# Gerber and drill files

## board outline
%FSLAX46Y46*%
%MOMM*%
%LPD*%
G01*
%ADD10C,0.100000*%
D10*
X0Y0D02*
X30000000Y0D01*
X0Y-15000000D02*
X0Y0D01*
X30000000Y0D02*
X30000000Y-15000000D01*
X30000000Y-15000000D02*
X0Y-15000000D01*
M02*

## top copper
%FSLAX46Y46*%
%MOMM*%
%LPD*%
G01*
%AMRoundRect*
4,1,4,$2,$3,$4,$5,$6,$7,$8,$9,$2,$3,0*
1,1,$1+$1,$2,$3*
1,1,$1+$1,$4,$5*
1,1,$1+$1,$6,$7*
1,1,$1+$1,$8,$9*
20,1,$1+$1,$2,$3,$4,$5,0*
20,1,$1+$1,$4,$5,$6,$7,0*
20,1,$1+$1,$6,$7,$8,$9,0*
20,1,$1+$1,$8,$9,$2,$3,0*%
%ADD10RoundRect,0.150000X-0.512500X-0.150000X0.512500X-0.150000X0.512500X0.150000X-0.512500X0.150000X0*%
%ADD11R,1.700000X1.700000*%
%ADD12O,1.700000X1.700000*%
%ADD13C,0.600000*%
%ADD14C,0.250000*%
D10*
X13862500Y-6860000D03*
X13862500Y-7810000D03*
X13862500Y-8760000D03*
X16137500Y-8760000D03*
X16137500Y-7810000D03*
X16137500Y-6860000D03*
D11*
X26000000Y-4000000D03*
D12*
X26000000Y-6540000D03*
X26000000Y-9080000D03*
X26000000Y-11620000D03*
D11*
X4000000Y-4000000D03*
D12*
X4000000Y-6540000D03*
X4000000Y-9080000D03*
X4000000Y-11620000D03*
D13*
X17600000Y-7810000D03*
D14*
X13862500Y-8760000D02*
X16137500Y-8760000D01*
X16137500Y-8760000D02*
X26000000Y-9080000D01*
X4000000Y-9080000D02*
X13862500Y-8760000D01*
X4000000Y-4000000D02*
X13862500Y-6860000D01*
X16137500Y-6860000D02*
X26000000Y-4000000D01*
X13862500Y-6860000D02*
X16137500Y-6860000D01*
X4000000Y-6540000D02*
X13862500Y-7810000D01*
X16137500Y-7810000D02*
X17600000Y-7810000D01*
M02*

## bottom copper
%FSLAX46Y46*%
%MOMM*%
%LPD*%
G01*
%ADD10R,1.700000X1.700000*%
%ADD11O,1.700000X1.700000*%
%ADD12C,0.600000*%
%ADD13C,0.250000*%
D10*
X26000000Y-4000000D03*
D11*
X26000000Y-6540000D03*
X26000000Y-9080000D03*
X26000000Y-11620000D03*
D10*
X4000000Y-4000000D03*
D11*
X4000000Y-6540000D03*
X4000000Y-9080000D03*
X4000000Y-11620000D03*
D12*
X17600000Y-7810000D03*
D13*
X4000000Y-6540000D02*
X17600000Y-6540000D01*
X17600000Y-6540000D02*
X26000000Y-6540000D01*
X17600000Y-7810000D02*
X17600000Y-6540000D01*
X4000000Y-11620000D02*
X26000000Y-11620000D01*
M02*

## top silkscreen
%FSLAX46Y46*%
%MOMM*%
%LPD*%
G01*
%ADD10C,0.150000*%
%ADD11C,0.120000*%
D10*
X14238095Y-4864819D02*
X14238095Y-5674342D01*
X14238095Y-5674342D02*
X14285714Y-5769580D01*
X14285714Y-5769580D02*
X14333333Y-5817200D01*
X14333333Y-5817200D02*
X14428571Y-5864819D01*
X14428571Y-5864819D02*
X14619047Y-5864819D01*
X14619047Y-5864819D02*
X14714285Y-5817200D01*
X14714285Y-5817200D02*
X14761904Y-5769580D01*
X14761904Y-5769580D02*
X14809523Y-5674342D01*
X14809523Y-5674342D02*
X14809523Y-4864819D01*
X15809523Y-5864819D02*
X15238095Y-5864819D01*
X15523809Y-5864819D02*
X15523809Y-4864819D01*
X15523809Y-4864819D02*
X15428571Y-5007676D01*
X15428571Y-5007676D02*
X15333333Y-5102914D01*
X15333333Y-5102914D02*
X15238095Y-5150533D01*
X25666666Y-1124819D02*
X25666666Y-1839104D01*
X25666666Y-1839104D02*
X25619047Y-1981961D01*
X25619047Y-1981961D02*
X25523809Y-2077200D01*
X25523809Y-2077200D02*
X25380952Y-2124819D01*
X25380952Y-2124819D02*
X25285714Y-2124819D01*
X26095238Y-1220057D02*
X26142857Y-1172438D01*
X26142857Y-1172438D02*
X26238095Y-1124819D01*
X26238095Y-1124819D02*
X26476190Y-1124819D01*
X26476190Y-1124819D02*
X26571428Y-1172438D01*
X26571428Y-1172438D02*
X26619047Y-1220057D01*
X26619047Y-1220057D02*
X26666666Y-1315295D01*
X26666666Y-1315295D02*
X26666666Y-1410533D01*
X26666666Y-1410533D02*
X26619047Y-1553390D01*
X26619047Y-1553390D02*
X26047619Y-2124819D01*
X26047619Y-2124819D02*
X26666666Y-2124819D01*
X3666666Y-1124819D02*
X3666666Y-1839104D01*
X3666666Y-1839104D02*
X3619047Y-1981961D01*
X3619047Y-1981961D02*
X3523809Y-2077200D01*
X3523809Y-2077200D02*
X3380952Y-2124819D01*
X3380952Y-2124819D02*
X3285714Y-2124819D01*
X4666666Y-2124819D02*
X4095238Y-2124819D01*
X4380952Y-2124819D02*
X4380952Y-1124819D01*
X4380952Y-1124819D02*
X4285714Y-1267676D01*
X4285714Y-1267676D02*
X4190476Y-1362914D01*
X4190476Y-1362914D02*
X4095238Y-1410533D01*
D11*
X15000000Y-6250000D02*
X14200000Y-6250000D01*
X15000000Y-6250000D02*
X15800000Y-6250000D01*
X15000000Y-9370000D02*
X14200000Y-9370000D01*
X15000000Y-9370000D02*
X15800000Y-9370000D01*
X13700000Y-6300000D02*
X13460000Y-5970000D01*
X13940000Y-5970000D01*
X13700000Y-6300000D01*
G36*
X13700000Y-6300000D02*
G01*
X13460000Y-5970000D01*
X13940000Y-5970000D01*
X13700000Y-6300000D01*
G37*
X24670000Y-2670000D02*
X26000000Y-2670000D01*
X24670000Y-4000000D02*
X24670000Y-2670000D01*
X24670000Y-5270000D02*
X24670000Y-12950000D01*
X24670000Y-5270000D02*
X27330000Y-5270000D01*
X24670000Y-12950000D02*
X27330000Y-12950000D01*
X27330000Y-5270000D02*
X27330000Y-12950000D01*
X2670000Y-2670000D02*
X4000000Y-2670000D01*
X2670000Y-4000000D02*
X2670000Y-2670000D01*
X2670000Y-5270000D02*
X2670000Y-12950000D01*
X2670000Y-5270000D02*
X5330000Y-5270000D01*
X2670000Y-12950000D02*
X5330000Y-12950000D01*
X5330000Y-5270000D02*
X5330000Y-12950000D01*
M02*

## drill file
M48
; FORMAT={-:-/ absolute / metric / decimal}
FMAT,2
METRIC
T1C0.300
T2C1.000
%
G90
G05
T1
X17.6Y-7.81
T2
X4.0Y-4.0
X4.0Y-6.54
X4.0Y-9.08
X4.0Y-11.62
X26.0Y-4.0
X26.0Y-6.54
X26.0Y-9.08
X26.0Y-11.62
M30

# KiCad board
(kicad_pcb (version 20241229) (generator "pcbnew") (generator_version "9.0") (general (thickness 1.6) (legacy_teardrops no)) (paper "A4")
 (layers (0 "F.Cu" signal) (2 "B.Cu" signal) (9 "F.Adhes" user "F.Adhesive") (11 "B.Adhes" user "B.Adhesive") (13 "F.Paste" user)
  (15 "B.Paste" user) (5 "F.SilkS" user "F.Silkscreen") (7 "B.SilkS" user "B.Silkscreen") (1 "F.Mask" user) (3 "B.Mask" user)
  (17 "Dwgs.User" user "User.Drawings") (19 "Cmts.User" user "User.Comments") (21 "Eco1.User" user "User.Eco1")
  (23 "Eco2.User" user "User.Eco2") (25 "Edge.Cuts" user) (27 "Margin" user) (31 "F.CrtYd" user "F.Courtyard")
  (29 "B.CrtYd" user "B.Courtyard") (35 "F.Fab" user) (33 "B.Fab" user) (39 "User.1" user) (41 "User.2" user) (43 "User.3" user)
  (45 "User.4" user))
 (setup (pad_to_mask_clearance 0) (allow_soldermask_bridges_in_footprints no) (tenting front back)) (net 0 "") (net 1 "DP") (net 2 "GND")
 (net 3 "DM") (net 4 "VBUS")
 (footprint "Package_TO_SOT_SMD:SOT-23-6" (layer "F.Cu") (at 15 7.81)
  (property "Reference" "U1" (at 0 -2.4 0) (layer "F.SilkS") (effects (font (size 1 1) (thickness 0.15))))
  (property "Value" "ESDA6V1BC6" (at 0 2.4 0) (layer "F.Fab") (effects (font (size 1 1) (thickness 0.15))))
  (fp_line (start 0 -1.56) (end -0.8 -1.56) (stroke (width 0.12) (type solid)) (layer "F.SilkS"))
  (fp_line (start 0 -1.56) (end 0.8 -1.56) (stroke (width 0.12) (type solid)) (layer "F.SilkS"))
  (fp_line (start 0 1.56) (end -0.8 1.56) (stroke (width 0.12) (type solid)) (layer "F.SilkS"))
  (fp_line (start 0 1.56) (end 0.8 1.56) (stroke (width 0.12) (type solid)) (layer "F.SilkS"))
  (fp_poly
   (pts (xy -1.3 -1.51) (xy -1.54 -1.84) (xy -1.06 -1.84) (xy -1.3 -1.51)) (stroke (width 0.12) (type solid)) (fill yes) (layer "F.SilkS"))
  (pad "1" smd roundrect (at -1.1375 -0.95) (size 1.325 0.6) (layers "F.Cu" "F.Mask" "F.Paste") (roundrect_rratio 0.25) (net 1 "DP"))
  (pad "2" smd roundrect (at -1.1375 0) (size 1.325 0.6) (layers "F.Cu" "F.Mask" "F.Paste") (roundrect_rratio 0.25) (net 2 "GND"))
  (pad "3" smd roundrect (at -1.1375 0.95) (size 1.325 0.6) (layers "F.Cu" "F.Mask" "F.Paste") (roundrect_rratio 0.25) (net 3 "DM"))
  (pad "4" smd roundrect (at 1.1375 0.95) (size 1.325 0.6) (layers "F.Cu" "F.Mask" "F.Paste") (roundrect_rratio 0.25) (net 3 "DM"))
  (pad "5" smd roundrect (at 1.1375 0) (size 1.325 0.6) (layers "F.Cu" "F.Mask" "F.Paste") (roundrect_rratio 0.25) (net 2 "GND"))
  (pad "6" smd roundrect (at 1.1375 -0.95) (size 1.325 0.6) (layers "F.Cu" "F.Mask" "F.Paste") (roundrect_rratio 0.25) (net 1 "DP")))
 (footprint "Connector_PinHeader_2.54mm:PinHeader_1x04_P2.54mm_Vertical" (layer "F.Cu") (at 26 4)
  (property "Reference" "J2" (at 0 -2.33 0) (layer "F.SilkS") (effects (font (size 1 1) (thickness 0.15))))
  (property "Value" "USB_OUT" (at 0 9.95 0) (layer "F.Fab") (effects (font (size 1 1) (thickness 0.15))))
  (fp_line (start -1.33 -1.33) (end 0 -1.33) (stroke (width 0.12) (type solid)) (layer "F.SilkS"))
  (fp_line (start -1.33 0) (end -1.33 -1.33) (stroke (width 0.12) (type solid)) (layer "F.SilkS"))
  (fp_line (start -1.33 1.27) (end -1.33 8.95) (stroke (width 0.12) (type solid)) (layer "F.SilkS"))
  (fp_line (start -1.33 1.27) (end 1.33 1.27) (stroke (width 0.12) (type solid)) (layer "F.SilkS"))
  (fp_line (start -1.33 8.95) (end 1.33 8.95) (stroke (width 0.12) (type solid)) (layer "F.SilkS"))
  (fp_line (start 1.33 1.27) (end 1.33 8.95) (stroke (width 0.12) (type solid)) (layer "F.SilkS"))
  (pad "1" thru_hole rect (at 0 0) (size 1.7 1.7) (drill 1) (layers "*.Cu" "*.Mask") (remove_unused_layers no) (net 1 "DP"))
  (pad "2" thru_hole oval (at 0 2.54) (size 1.7 1.7) (drill 1) (layers "*.Cu" "*.Mask") (remove_unused_layers no) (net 2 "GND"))
  (pad "3" thru_hole oval (at 0 5.08) (size 1.7 1.7) (drill 1) (layers "*.Cu" "*.Mask") (remove_unused_layers no) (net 3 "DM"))
  (pad "4" thru_hole oval (at 0 7.62) (size 1.7 1.7) (drill 1) (layers "*.Cu" "*.Mask") (remove_unused_layers no) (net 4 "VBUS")))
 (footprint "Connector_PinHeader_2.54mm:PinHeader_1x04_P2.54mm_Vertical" (layer "F.Cu") (at 4 4)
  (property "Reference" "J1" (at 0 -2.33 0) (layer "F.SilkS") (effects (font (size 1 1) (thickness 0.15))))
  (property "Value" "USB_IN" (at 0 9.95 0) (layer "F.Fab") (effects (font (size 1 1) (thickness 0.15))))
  (fp_line (start -1.33 -1.33) (end 0 -1.33) (stroke (width 0.12) (type solid)) (layer "F.SilkS"))
  (fp_line (start -1.33 0) (end -1.33 -1.33) (stroke (width 0.12) (type solid)) (layer "F.SilkS"))
  (fp_line (start -1.33 1.27) (end -1.33 8.95) (stroke (width 0.12) (type solid)) (layer "F.SilkS"))
  (fp_line (start -1.33 1.27) (end 1.33 1.27) (stroke (width 0.12) (type solid)) (layer "F.SilkS"))
  (fp_line (start -1.33 8.95) (end 1.33 8.95) (stroke (width 0.12) (type solid)) (layer "F.SilkS"))
  (fp_line (start 1.33 1.27) (end 1.33 8.95) (stroke (width 0.12) (type solid)) (layer "F.SilkS"))
  (pad "1" thru_hole rect (at 0 0) (size 1.7 1.7) (drill 1) (layers "*.Cu" "*.Mask") (remove_unused_layers no) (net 1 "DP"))
  (pad "2" thru_hole oval (at 0 2.54) (size 1.7 1.7) (drill 1) (layers "*.Cu" "*.Mask") (remove_unused_layers no) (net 2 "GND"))
  (pad "3" thru_hole oval (at 0 5.08) (size 1.7 1.7) (drill 1) (layers "*.Cu" "*.Mask") (remove_unused_layers no) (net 3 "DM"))
  (pad "4" thru_hole oval (at 0 7.62) (size 1.7 1.7) (drill 1) (layers "*.Cu" "*.Mask") (remove_unused_layers no) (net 4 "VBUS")))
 (gr_line (start 0 0) (end 30 0) (stroke (width 0.1) (type default)) (layer "Edge.Cuts"))
 (gr_line (start 0 15) (end 0 0) (stroke (width 0.1) (type default)) (layer "Edge.Cuts"))
 (gr_line (start 30 0) (end 30 15) (stroke (width 0.1) (type default)) (layer "Edge.Cuts"))
 (gr_line (start 30 15) (end 0 15) (stroke (width 0.1) (type default)) (layer "Edge.Cuts"))
 (segment (start 13.8625 8.76) (end 16.1375 8.76) (width 0.25) (layer "F.Cu") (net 3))
 (segment (start 16.1375 8.76) (end 26 9.08) (width 0.25) (layer "F.Cu") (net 3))
 (segment (start 4 9.08) (end 13.8625 8.76) (width 0.25) (layer "F.Cu") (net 3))
 (segment (start 4 4) (end 13.8625 6.86) (width 0.25) (layer "F.Cu") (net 1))
 (segment (start 16.1375 6.86) (end 26 4) (width 0.25) (layer "F.Cu") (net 1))
 (segment (start 13.8625 6.86) (end 16.1375 6.86) (width 0.25) (layer "F.Cu") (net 1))
 (segment (start 4 6.54) (end 13.8625 7.81) (width 0.25) (layer "F.Cu") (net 2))
 (segment (start 16.1375 7.81) (end 17.6 7.81) (width 0.25) (layer "F.Cu") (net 2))
 (via (at 17.6 7.81) (size 0.6) (drill 0.3) (layers "F.Cu" "B.Cu") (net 2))
 (segment (start 4 6.54) (end 17.6 6.54) (width 0.25) (layer "B.Cu") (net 2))
 (segment (start 17.6 6.54) (end 26 6.54) (width 0.25) (layer "B.Cu") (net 2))
 (segment (start 17.6 7.81) (end 17.6 6.54) (width 0.25) (layer "B.Cu") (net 2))
 (segment (start 4 11.62) (end 26 11.62) (width 0.25) (layer "B.Cu") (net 4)))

